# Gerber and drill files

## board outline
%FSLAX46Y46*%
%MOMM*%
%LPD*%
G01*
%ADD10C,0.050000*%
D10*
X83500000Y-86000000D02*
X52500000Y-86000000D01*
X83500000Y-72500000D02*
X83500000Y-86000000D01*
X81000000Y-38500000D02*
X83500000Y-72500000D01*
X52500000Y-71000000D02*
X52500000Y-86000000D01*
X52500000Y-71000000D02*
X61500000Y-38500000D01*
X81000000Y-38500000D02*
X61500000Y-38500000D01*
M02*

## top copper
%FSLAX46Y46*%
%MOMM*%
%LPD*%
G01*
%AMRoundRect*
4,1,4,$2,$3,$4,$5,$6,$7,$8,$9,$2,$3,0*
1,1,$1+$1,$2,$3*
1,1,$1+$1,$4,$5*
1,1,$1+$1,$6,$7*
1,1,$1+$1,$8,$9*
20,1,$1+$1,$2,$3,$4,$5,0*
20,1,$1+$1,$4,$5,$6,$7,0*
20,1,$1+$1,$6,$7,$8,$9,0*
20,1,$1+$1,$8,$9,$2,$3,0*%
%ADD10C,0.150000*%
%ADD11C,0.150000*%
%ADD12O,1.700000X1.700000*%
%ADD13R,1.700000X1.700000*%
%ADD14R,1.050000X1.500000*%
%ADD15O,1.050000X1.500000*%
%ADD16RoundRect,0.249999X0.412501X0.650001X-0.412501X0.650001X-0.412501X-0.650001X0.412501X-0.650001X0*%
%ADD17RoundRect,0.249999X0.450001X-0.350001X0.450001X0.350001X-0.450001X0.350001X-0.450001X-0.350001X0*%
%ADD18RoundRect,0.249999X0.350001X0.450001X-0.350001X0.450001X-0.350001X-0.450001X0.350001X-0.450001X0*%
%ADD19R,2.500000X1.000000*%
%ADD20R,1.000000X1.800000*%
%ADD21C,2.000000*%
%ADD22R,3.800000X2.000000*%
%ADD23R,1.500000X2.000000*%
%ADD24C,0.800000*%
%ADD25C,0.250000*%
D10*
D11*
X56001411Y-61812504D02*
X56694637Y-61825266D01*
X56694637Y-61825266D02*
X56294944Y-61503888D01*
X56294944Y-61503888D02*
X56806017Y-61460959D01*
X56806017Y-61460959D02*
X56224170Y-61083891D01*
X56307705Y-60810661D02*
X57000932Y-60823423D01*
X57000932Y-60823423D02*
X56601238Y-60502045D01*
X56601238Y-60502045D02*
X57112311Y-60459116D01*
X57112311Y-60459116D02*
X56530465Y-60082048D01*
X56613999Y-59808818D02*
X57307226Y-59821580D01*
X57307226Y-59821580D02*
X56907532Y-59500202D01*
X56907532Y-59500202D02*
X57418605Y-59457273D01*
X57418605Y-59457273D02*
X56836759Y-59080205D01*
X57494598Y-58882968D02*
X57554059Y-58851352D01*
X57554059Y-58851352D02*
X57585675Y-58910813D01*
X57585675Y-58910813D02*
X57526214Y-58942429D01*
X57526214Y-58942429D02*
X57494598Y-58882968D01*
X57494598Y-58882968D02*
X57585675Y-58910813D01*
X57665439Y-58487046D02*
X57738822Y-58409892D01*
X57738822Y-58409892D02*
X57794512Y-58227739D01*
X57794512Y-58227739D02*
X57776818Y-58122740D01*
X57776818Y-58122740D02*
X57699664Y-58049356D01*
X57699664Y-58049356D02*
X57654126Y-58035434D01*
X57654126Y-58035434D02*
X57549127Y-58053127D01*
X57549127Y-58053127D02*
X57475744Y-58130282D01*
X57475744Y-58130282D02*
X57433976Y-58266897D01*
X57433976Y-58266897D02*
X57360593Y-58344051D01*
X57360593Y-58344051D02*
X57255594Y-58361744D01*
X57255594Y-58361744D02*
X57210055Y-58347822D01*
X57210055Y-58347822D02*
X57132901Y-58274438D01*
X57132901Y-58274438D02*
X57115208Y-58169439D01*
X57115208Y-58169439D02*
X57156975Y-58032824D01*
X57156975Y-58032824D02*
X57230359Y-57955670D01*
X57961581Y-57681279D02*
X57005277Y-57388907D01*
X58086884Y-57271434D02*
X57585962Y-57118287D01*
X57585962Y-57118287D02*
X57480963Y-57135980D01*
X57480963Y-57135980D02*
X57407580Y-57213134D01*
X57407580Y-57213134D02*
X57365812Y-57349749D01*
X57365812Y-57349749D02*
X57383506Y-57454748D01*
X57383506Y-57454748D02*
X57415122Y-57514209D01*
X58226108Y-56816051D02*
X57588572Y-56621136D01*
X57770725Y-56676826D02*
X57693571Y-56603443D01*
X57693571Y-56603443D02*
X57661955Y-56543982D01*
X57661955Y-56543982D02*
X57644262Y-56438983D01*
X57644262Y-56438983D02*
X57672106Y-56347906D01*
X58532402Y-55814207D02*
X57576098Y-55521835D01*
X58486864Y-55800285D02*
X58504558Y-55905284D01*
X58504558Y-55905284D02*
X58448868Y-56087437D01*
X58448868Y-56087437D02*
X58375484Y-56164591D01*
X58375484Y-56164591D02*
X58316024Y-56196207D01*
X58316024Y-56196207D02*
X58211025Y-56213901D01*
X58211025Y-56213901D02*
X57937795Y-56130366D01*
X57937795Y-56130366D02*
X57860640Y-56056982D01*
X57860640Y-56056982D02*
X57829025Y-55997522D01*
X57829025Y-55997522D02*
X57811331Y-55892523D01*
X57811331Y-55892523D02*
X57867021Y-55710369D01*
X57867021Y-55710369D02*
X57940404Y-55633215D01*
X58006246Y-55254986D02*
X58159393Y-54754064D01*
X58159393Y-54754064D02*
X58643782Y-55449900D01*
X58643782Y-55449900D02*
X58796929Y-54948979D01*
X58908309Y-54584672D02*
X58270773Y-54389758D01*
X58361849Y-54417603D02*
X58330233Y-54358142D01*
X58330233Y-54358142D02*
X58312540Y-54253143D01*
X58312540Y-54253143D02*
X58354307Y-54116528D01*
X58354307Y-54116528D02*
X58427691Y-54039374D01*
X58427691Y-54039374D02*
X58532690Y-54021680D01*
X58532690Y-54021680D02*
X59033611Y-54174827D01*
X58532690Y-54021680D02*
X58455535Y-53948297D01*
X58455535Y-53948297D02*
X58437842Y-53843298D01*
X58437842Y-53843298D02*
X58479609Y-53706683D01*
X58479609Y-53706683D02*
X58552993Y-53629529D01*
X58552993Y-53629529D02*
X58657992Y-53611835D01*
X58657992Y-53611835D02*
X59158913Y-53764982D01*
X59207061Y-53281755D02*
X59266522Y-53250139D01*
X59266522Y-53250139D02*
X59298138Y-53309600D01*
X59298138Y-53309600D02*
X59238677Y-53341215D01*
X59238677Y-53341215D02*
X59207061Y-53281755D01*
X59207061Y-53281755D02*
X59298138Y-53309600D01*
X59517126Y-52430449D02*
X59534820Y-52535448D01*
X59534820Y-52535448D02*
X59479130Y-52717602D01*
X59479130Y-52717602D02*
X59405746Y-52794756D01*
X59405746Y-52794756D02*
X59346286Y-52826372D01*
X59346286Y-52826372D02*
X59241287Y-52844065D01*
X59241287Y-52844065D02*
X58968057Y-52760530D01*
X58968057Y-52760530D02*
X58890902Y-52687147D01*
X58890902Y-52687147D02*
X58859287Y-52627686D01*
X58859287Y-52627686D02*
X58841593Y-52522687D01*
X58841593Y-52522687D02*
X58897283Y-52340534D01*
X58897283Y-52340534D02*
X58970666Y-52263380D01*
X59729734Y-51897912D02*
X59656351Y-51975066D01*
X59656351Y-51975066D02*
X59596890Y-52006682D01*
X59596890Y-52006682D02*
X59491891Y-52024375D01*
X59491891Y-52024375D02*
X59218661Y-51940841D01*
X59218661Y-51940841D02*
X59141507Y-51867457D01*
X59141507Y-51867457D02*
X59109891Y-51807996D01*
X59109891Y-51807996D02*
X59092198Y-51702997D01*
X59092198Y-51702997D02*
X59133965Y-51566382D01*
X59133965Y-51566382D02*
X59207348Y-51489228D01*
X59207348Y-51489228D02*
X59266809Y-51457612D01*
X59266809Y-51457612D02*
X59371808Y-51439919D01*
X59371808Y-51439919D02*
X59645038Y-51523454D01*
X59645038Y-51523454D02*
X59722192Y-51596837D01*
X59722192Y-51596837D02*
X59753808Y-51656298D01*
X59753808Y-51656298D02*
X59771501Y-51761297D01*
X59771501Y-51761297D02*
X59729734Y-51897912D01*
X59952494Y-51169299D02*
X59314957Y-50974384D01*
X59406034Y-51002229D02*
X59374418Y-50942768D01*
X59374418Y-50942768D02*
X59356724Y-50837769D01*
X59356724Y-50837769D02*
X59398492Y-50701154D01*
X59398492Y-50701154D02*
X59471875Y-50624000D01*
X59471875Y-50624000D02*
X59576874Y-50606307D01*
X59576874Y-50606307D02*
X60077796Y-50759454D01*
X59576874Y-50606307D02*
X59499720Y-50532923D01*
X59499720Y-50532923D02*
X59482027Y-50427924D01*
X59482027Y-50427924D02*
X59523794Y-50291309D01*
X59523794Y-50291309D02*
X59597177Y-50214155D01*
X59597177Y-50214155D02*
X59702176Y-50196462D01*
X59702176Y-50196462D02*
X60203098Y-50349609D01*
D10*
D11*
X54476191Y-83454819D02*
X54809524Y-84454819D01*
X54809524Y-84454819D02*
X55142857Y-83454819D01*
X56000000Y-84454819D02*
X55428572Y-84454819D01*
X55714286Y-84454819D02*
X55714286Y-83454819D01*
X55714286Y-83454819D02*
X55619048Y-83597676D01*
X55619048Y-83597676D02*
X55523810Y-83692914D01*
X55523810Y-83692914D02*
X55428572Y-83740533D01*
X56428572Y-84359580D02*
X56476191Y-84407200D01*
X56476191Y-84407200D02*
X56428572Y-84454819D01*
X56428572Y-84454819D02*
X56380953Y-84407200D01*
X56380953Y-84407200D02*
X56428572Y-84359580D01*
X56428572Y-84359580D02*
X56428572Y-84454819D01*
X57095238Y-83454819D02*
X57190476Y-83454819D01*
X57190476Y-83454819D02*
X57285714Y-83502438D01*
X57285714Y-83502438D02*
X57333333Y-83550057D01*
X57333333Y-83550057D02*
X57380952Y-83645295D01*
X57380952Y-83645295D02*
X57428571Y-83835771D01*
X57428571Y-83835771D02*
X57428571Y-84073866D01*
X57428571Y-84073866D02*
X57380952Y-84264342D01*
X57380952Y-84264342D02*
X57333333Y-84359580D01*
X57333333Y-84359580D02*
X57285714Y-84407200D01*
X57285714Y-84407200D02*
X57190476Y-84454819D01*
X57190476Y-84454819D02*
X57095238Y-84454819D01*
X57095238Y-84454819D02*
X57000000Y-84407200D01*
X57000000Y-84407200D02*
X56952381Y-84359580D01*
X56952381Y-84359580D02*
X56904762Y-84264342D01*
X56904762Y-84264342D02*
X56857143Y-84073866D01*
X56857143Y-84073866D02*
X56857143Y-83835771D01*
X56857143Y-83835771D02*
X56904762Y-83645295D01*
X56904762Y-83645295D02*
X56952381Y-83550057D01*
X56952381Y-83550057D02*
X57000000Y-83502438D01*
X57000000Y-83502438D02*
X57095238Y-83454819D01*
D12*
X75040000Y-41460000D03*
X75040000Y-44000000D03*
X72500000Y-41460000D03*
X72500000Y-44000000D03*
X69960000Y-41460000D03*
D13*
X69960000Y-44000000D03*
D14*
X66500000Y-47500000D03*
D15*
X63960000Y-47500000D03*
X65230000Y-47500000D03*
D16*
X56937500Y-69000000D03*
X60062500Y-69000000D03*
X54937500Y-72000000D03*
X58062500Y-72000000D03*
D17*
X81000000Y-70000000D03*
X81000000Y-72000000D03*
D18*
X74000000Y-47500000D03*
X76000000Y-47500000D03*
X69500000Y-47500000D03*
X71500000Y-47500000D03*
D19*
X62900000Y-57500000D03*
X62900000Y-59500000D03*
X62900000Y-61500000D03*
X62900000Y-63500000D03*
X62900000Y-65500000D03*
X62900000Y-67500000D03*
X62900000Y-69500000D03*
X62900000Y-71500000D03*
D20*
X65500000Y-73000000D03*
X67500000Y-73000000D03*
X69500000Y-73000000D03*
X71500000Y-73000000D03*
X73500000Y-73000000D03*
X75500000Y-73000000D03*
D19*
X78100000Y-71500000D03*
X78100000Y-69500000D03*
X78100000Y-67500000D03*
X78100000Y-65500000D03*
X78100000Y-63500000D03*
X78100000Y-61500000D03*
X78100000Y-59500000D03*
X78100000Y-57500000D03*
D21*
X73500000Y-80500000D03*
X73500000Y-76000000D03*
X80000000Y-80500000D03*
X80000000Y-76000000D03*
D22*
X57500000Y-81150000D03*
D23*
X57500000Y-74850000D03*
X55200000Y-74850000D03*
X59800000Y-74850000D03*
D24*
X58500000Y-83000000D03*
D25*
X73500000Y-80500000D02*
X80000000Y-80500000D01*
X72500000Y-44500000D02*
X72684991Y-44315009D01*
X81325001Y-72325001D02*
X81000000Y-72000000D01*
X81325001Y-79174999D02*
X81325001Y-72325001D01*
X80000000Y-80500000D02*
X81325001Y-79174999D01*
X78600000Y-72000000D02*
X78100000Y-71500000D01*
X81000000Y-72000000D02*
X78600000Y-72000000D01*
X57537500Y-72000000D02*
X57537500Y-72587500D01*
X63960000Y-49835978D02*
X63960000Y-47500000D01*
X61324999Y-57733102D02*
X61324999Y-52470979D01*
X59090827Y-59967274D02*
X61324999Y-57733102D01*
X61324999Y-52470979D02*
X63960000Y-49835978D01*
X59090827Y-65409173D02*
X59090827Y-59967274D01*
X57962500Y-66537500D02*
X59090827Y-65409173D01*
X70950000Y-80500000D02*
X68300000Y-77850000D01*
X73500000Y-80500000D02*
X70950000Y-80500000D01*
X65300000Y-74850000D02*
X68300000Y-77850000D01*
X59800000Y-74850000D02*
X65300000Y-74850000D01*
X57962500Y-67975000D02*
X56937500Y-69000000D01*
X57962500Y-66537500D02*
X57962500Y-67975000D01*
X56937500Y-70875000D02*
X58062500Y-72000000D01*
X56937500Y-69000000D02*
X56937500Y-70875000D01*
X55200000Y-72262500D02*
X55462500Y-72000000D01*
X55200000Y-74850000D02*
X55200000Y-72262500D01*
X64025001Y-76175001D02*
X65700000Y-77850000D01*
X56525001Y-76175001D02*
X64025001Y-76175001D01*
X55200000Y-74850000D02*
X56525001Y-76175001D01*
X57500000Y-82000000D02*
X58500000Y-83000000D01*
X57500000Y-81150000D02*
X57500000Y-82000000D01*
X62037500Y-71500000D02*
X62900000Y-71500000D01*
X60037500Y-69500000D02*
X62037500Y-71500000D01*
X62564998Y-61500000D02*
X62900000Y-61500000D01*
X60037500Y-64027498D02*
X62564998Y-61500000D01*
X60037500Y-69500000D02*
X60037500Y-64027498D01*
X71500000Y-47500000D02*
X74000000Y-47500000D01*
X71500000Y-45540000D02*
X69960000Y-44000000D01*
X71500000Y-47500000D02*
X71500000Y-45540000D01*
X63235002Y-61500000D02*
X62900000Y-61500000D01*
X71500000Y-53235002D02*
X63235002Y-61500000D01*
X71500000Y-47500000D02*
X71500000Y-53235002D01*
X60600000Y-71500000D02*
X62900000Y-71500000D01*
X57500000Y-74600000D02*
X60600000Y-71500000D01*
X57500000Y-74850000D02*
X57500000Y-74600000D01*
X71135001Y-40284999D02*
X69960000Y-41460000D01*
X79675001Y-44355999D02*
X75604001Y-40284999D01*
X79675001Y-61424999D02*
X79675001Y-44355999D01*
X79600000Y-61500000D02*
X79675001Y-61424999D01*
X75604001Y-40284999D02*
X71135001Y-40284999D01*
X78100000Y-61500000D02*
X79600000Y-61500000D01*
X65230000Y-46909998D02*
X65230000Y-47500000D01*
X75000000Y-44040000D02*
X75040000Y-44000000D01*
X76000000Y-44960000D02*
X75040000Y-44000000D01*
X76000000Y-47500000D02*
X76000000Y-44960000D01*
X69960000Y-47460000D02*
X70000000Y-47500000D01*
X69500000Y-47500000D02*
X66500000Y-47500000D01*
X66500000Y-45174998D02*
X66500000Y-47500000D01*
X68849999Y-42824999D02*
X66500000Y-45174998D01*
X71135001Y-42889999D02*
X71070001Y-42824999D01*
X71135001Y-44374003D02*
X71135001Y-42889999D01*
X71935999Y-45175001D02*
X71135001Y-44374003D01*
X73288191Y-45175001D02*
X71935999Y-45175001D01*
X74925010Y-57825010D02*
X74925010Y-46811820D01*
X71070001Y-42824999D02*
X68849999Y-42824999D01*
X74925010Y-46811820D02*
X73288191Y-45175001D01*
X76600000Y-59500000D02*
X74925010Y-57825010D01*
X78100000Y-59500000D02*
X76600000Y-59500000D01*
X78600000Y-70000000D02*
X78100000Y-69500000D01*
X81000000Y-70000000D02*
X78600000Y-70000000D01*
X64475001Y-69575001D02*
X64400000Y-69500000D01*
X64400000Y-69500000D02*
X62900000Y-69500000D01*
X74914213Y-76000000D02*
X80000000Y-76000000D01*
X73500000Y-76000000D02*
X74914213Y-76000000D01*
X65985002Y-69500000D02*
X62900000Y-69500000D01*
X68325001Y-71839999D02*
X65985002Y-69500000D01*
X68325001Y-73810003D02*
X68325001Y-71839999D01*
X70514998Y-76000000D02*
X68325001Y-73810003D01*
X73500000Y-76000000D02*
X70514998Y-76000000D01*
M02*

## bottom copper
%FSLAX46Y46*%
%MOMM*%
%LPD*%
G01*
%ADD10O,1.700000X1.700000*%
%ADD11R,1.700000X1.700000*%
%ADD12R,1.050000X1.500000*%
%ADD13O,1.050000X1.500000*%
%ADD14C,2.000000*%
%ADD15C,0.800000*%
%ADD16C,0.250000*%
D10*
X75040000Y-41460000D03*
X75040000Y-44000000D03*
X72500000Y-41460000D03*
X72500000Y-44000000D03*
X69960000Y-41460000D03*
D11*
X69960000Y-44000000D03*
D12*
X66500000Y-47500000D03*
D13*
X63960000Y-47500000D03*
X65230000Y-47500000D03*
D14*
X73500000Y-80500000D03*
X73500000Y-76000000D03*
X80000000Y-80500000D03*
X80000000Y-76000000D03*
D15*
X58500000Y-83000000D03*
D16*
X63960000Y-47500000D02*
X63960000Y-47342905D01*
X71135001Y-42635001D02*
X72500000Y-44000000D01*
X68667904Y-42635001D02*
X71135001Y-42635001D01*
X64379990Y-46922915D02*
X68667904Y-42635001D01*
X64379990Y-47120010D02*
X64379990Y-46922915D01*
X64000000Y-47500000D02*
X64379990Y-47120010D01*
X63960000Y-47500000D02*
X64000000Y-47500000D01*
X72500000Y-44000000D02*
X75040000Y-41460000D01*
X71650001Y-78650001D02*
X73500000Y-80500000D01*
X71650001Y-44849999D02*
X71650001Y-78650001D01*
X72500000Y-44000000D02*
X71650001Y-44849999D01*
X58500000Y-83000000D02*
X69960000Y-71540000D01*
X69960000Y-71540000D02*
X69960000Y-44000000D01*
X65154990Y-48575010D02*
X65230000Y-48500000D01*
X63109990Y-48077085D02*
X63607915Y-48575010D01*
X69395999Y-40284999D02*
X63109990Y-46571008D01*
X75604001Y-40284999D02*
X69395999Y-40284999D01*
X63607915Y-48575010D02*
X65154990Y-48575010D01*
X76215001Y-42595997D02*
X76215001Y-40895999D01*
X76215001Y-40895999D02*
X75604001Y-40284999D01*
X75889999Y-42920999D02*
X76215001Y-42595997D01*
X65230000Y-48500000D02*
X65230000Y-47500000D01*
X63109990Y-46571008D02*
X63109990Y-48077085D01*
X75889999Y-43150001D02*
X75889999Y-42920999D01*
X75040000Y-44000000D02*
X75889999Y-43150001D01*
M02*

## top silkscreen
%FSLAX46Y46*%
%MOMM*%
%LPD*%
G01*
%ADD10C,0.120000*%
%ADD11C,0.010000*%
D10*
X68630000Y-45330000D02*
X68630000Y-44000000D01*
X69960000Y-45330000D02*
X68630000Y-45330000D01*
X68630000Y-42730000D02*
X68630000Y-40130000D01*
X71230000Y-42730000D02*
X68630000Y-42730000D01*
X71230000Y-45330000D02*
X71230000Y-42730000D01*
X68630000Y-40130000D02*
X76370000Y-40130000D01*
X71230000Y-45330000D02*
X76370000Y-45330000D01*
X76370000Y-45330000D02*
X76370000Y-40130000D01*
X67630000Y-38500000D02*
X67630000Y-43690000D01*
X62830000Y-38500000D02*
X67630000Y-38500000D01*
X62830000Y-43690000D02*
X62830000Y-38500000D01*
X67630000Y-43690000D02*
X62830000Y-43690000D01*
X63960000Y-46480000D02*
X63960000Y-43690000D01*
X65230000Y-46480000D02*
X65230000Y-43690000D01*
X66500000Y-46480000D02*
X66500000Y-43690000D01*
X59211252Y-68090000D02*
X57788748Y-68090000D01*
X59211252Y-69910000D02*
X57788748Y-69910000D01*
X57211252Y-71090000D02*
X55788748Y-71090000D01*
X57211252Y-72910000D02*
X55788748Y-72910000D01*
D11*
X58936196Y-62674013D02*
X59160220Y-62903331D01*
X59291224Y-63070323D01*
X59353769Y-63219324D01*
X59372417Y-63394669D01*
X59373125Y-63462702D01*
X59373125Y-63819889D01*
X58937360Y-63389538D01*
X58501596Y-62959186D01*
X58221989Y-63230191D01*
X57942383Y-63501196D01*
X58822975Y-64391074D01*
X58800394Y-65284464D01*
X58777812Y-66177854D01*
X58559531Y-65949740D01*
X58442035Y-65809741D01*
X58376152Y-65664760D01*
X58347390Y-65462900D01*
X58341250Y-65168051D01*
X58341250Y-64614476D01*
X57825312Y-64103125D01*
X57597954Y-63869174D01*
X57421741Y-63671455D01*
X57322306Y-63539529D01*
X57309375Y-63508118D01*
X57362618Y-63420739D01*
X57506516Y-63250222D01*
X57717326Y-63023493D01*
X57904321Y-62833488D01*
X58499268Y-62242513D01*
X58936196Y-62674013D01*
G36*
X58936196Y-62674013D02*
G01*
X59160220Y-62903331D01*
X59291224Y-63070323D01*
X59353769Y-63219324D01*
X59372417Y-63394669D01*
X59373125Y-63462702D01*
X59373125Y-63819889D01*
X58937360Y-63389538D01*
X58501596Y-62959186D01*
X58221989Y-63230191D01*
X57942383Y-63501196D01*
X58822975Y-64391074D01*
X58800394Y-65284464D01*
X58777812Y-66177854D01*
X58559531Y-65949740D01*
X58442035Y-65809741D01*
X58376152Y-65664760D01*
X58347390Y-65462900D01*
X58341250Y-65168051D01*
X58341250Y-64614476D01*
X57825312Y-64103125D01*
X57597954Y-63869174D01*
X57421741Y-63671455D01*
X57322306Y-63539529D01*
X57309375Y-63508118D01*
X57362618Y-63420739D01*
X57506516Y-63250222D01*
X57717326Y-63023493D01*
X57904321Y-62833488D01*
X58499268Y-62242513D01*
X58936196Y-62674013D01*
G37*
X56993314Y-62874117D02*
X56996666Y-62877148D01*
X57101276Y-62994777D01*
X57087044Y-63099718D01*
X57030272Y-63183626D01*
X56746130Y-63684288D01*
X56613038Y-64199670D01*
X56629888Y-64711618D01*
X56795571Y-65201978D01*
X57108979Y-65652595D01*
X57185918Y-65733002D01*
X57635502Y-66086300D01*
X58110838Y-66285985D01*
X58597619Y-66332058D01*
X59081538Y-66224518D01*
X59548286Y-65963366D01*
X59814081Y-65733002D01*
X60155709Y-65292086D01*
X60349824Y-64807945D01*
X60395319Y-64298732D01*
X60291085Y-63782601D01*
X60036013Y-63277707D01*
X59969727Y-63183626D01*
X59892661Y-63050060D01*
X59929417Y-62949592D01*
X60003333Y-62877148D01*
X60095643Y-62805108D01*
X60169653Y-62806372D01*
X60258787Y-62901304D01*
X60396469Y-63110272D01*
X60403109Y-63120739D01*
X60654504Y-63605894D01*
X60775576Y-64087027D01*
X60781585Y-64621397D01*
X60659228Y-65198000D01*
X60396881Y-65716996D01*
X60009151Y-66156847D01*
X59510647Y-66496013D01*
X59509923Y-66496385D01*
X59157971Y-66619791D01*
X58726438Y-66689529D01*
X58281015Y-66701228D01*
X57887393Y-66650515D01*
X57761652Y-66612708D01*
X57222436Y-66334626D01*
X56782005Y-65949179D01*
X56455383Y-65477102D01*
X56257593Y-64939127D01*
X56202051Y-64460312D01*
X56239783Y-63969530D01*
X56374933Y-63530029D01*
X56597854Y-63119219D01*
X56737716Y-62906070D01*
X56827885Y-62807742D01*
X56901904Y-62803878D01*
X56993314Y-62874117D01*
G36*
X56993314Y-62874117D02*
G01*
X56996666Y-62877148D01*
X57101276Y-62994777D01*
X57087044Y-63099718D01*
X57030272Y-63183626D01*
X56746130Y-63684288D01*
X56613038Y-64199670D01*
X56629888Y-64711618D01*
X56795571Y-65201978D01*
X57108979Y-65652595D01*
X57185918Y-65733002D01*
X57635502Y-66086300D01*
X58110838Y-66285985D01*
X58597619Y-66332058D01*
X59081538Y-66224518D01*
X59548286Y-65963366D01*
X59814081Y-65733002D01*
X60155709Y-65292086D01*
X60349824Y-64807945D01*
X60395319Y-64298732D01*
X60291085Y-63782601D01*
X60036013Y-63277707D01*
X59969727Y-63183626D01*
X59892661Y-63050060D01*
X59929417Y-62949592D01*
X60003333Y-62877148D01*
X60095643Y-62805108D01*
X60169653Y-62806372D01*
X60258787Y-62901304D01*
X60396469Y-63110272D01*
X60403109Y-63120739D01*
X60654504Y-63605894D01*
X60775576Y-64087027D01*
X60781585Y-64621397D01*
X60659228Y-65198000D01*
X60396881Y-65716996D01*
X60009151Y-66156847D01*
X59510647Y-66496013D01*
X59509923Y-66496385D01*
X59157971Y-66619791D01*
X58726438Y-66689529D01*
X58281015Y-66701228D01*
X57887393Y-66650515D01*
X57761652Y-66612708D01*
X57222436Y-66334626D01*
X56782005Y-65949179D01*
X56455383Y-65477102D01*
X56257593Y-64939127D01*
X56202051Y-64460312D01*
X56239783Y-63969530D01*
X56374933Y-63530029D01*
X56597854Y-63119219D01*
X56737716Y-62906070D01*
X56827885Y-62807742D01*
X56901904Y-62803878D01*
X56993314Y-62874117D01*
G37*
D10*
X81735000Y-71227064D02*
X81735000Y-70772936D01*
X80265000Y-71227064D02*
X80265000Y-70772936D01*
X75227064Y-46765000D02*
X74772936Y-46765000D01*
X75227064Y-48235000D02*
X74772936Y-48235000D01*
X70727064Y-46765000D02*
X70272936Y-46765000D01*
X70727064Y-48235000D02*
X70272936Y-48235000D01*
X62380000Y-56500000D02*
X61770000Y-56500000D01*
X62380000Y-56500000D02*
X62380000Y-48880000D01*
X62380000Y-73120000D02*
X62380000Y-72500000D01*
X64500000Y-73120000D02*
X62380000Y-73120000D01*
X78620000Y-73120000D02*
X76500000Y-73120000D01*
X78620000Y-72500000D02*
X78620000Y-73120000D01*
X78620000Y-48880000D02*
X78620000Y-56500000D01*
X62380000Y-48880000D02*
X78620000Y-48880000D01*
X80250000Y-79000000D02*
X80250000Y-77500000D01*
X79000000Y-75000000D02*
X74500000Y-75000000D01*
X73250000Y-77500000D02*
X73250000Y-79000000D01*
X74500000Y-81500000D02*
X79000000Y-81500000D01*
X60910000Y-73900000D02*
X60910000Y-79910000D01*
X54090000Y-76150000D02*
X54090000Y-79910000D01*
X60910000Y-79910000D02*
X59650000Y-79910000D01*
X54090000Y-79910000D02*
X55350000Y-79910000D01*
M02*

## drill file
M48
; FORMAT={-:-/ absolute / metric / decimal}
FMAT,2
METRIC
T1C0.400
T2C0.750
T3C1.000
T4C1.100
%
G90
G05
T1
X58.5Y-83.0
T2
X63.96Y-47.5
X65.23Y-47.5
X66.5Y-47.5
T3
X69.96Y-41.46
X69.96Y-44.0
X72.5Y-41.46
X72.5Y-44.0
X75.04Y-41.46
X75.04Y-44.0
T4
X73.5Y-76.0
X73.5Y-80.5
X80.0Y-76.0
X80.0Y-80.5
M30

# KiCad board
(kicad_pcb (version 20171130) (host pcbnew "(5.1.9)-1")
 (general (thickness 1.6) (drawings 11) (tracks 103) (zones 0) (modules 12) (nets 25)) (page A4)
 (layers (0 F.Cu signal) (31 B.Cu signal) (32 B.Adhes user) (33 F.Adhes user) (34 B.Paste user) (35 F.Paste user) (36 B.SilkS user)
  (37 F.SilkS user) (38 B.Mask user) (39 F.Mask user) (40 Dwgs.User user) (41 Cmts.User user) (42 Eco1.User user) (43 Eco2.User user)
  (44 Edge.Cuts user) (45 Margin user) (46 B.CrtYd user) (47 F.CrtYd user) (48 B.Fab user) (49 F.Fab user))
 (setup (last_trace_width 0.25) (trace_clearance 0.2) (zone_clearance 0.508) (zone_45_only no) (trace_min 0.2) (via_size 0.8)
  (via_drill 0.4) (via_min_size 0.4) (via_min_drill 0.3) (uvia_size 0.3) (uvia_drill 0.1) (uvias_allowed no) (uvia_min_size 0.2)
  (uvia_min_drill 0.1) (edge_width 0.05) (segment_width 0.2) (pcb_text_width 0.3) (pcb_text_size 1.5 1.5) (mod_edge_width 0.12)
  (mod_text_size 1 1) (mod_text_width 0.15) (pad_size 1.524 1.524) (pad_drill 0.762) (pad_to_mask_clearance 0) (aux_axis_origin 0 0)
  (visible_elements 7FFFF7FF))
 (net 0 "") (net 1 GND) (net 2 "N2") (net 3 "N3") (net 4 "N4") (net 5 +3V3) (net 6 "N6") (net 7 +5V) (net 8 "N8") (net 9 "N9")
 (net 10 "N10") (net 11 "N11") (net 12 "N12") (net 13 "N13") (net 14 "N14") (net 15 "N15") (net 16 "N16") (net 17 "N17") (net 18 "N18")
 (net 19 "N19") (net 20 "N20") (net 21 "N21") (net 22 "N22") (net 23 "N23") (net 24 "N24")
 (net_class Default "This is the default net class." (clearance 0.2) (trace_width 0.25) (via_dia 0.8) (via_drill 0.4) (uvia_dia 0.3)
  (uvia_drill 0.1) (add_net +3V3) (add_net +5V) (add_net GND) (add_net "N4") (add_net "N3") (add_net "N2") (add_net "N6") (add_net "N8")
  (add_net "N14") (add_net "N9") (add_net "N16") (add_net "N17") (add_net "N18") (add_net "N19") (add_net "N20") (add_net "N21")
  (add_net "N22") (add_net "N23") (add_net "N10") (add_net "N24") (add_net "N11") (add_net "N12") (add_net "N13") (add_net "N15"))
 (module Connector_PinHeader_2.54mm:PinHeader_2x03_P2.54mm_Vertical (layer F.Cu) (at 69.96 44 90)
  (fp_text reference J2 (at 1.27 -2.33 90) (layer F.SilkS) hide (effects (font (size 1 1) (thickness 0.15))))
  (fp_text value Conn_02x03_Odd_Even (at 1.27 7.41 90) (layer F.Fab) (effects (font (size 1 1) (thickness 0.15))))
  (fp_line (start -1.33 -1.33) (end 0 -1.33) (layer F.SilkS) (width 0.12))
  (fp_line (start -1.33 0) (end -1.33 -1.33) (layer F.SilkS) (width 0.12))
  (fp_line (start 1.27 -1.33) (end 3.87 -1.33) (layer F.SilkS) (width 0.12))
  (fp_line (start 1.27 1.27) (end 1.27 -1.33) (layer F.SilkS) (width 0.12))
  (fp_line (start -1.33 1.27) (end 1.27 1.27) (layer F.SilkS) (width 0.12))
  (fp_line (start 3.87 -1.33) (end 3.87 6.41) (layer F.SilkS) (width 0.12))
  (fp_line (start -1.33 1.27) (end -1.33 6.41) (layer F.SilkS) (width 0.12))
  (fp_line (start -1.33 6.41) (end 3.87 6.41) (layer F.SilkS) (width 0.12))
  (pad 6 thru_hole oval (at 2.54 5.08 90) (size 1.7 1.7) (drill 1) (layers *.Cu *.Mask) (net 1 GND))
  (pad 5 thru_hole oval (at 0 5.08 90) (size 1.7 1.7) (drill 1) (layers *.Cu *.Mask) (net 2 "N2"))
  (pad 4 thru_hole oval (at 2.54 2.54 90) (size 1.7 1.7) (drill 1) (layers *.Cu *.Mask) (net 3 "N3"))
  (pad 3 thru_hole oval (at 0 2.54 90) (size 1.7 1.7) (drill 1) (layers *.Cu *.Mask) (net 1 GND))
  (pad 2 thru_hole oval (at 2.54 0 90) (size 1.7 1.7) (drill 1) (layers *.Cu *.Mask) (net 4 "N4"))
  (pad 1 thru_hole rect (at 0 0 90) (size 1.7 1.7) (drill 1) (layers *.Cu *.Mask) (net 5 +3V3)))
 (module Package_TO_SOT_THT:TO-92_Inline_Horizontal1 (layer F.Cu) (at 66.5 47.5 180)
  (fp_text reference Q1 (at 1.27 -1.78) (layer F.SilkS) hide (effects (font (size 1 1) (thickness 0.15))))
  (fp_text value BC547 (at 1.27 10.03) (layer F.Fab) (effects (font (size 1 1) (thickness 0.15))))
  (fp_line (start -1.13 9) (end -1.13 3.81) (layer F.SilkS) (width 0.12))
  (fp_line (start 3.67 9) (end -1.13 9) (layer F.SilkS) (width 0.12))
  (fp_line (start 3.67 3.81) (end 3.67 9) (layer F.SilkS) (width 0.12))
  (fp_line (start -1.13 3.81) (end 3.67 3.81) (layer F.SilkS) (width 0.12))
  (fp_line (start 2.54 1.02) (end 2.54 3.81) (layer F.SilkS) (width 0.12))
  (fp_line (start 1.27 1.02) (end 1.27 3.81) (layer F.SilkS) (width 0.12))
  (fp_line (start 0 1.02) (end 0 3.81) (layer F.SilkS) (width 0.12))
  (pad 1 thru_hole rect (at 0 0 180) (size 1.05 1.5) (drill 0.75) (layers *.Cu *.Mask) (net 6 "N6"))
  (pad 3 thru_hole oval (at 2.54 0 180) (size 1.05 1.5) (drill 0.75) (layers *.Cu *.Mask) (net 1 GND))
  (pad 2 thru_hole oval (at 1.27 0 180) (size 1.05 1.5) (drill 0.75) (layers *.Cu *.Mask) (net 2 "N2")))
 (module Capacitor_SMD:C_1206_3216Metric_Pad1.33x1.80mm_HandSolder (layer F.Cu) (at 58.5 69 180)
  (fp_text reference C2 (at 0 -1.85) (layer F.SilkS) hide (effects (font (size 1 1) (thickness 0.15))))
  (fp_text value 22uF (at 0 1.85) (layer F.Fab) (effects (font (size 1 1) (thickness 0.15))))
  (fp_line (start -0.711252 0.91) (end 0.711252 0.91) (layer F.SilkS) (width 0.12))
  (fp_line (start -0.711252 -0.91) (end 0.711252 -0.91) (layer F.SilkS) (width 0.12))
  (pad 2 smd roundrect (at 1.5625 0 180) (size 1.325 1.8) (layers F.Cu F.Paste F.Mask) (roundrect_rratio 0.1886784905660377) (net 1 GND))
  (pad 1 smd roundrect (at -1.5625 0 180) (size 1.325 1.8) (layers F.Cu F.Paste F.Mask) (roundrect_rratio 0.1886784905660377) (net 5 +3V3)))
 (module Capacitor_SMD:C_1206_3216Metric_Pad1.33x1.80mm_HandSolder (layer F.Cu) (at 56.5 72 180)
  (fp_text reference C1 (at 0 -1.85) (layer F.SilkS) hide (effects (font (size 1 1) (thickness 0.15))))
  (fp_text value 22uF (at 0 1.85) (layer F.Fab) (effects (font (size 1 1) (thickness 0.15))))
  (fp_line (start -0.711252 0.91) (end 0.711252 0.91) (layer F.SilkS) (width 0.12))
  (fp_line (start -0.711252 -0.91) (end 0.711252 -0.91) (layer F.SilkS) (width 0.12))
  (pad 2 smd roundrect (at 1.5625 0 180) (size 1.325 1.8) (layers F.Cu F.Paste F.Mask) (roundrect_rratio 0.1886784905660377) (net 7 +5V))
  (pad 1 smd roundrect (at -1.5625 0 180) (size 1.325 1.8) (layers F.Cu F.Paste F.Mask) (roundrect_rratio 0.1886784905660377) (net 1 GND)))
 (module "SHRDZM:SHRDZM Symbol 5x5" (layer F.Cu) (at 58.5 64.5)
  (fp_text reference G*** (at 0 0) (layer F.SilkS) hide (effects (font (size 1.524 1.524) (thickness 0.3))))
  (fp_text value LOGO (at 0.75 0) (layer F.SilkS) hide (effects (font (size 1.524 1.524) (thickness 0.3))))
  (fp_poly
   (pts (xy 0.436196 -1.825987) (xy 0.66022 -1.596669) (xy 0.791224 -1.429677) (xy 0.853769 -1.280676) (xy 0.872417 -1.105331)
    (xy 0.873125 -1.037298) (xy 0.873125 -0.680111) (xy 0.43736 -1.110462) (xy 0.001596 -1.540814) (xy -0.278011 -1.269809)
    (xy -0.557617 -0.998804) (xy 0.322975 -0.108926) (xy 0.300394 0.784464) (xy 0.277812 1.677854) (xy 0.059531 1.44974)
    (xy -0.057965 1.309741) (xy -0.123848 1.16476) (xy -0.15261 0.9629) (xy -0.15875 0.668051) (xy -0.15875 0.114476)
    (xy -0.674688 -0.396875) (xy -0.902046 -0.630826) (xy -1.078259 -0.828545) (xy -1.177694 -0.960471) (xy -1.190625 -0.991882)
    (xy -1.137382 -1.079261) (xy -0.993484 -1.249778) (xy -0.782674 -1.476507) (xy -0.595679 -1.666512) (xy -0.000732 -2.257487)
    (xy 0.436196 -1.825987))
   (layer F.SilkS) (width 0.01))
  (fp_poly
   (pts (xy -1.506686 -1.625883) (xy -1.503334 -1.622852) (xy -1.398724 -1.505223) (xy -1.412956 -1.400282) (xy -1.469728 -1.316374)
    (xy -1.75387 -0.815712) (xy -1.886962 -0.30033) (xy -1.870112 0.211618) (xy -1.704429 0.701978) (xy -1.391021 1.152595)
    (xy -1.314082 1.233002) (xy -0.864498 1.5863) (xy -0.389162 1.785985) (xy 0.097619 1.832058) (xy 0.581538 1.724518)
    (xy 1.048286 1.463366) (xy 1.314081 1.233002) (xy 1.655709 0.792086) (xy 1.849824 0.307945) (xy 1.895319 -0.201268)
    (xy 1.791085 -0.717399) (xy 1.536013 -1.222293) (xy 1.469727 -1.316374) (xy 1.392661 -1.44994) (xy 1.429417 -1.550408)
    (xy 1.503333 -1.622852) (xy 1.595643 -1.694892) (xy 1.669653 -1.693628) (xy 1.758787 -1.598696) (xy 1.896469 -1.389728)
    (xy 1.903109 -1.379261) (xy 2.154504 -0.894106) (xy 2.275576 -0.412973) (xy 2.281585 0.121397) (xy 2.159228 0.698)
    (xy 1.896881 1.216996) (xy 1.509151 1.656847) (xy 1.010647 1.996013) (xy 1.009923 1.996385) (xy 0.657971 2.119791)
    (xy 0.226438 2.189529) (xy -0.218985 2.201228) (xy -0.612607 2.150515) (xy -0.738348 2.112708) (xy -1.277564 1.834626)
    (xy -1.717995 1.449179) (xy -2.044617 0.977102) (xy -2.242407 0.439127) (xy -2.297949 -0.039688) (xy -2.260217 -0.53047)
    (xy -2.125067 -0.969971) (xy -1.902146 -1.380781) (xy -1.762284 -1.59393) (xy -1.672115 -1.692258) (xy -1.598096 -1.696122)
    (xy -1.506686 -1.625883))
   (layer F.SilkS) (width 0.01)))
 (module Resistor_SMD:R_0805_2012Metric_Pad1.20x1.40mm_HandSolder (layer F.Cu) (at 81 71 90)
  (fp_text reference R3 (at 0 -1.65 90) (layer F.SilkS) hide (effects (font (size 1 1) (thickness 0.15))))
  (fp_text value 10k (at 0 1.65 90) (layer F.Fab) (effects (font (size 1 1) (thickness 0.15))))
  (fp_line (start -0.227064 0.735) (end 0.227064 0.735) (layer F.SilkS) (width 0.12))
  (fp_line (start -0.227064 -0.735) (end 0.227064 -0.735) (layer F.SilkS) (width 0.12))
  (pad 2 smd roundrect (at 1 0 90) (size 1.2 1.4) (layers F.Cu F.Paste F.Mask) (roundrect_rratio 0.2083325) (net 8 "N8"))
  (pad 1 smd roundrect (at -1 0 90) (size 1.2 1.4) (layers F.Cu F.Paste F.Mask) (roundrect_rratio 0.2083325) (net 1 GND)))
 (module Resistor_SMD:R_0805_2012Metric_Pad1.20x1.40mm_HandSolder (layer F.Cu) (at 75 47.5 180)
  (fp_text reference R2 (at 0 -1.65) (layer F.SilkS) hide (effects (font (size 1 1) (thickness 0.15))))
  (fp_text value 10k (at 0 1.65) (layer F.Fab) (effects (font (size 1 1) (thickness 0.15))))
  (fp_line (start -0.227064 0.735) (end 0.227064 0.735) (layer F.SilkS) (width 0.12))
  (fp_line (start -0.227064 -0.735) (end 0.227064 -0.735) (layer F.SilkS) (width 0.12))
  (pad 2 smd roundrect (at 1 0 180) (size 1.2 1.4) (layers F.Cu F.Paste F.Mask) (roundrect_rratio 0.2083325) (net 5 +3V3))
  (pad 1 smd roundrect (at -1 0 180) (size 1.2 1.4) (layers F.Cu F.Paste F.Mask) (roundrect_rratio 0.2083325) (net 2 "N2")))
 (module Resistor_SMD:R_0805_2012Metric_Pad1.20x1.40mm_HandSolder (layer F.Cu) (at 70.5 47.5 180)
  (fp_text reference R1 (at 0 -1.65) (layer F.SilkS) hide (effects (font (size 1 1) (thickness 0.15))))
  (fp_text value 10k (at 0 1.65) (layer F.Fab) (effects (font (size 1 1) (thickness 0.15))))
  (fp_line (start -0.227064 0.735) (end 0.227064 0.735) (layer F.SilkS) (width 0.12))
  (fp_line (start -0.227064 -0.735) (end 0.227064 -0.735) (layer F.SilkS) (width 0.12))
  (pad 2 smd roundrect (at 1 0 180) (size 1.2 1.4) (layers F.Cu F.Paste F.Mask) (roundrect_rratio 0.2083325) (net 6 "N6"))
  (pad 1 smd roundrect (at -1 0 180) (size 1.2 1.4) (layers F.Cu F.Paste F.Mask) (roundrect_rratio 0.2083325) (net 5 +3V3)))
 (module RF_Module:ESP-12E (layer F.Cu) (at 70.5 61)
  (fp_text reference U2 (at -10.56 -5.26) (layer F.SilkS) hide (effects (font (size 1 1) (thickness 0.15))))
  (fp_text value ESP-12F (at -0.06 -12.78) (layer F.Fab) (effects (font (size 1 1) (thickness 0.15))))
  (fp_line (start -8.12 -4.5) (end -8.73 -4.5) (layer F.SilkS) (width 0.12))
  (fp_line (start -8.12 -4.5) (end -8.12 -12.12) (layer F.SilkS) (width 0.12))
  (fp_line (start -8.12 12.12) (end -8.12 11.5) (layer F.SilkS) (width 0.12))
  (fp_line (start -6 12.12) (end -8.12 12.12) (layer F.SilkS) (width 0.12))
  (fp_line (start 8.12 12.12) (end 6 12.12) (layer F.SilkS) (width 0.12))
  (fp_line (start 8.12 11.5) (end 8.12 12.12) (layer F.SilkS) (width 0.12))
  (fp_line (start 8.12 -12.12) (end 8.12 -4.5) (layer F.SilkS) (width 0.12))
  (fp_line (start -8.12 -12.12) (end 8.12 -12.12) (layer F.SilkS) (width 0.12))
  (pad 1 smd rect (at -7.6 -3.5) (size 2.5 1) (layers F.Cu F.Paste F.Mask) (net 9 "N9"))
  (pad 2 smd rect (at -7.6 -1.5) (size 2.5 1) (layers F.Cu F.Paste F.Mask) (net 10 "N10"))
  (pad 3 smd rect (at -7.6 0.5) (size 2.5 1) (layers F.Cu F.Paste F.Mask) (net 5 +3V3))
  (pad 4 smd rect (at -7.6 2.5) (size 2.5 1) (layers F.Cu F.Paste F.Mask) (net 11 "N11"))
  (pad 5 smd rect (at -7.6 4.5) (size 2.5 1) (layers F.Cu F.Paste F.Mask) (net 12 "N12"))
  (pad 6 smd rect (at -7.6 6.5) (size 2.5 1) (layers F.Cu F.Paste F.Mask) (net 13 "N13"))
  (pad 7 smd rect (at -7.6 8.5) (size 2.5 1) (layers F.Cu F.Paste F.Mask) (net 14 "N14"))
  (pad 8 smd rect (at -7.6 10.5) (size 2.5 1) (layers F.Cu F.Paste F.Mask) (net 5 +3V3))
  (pad 9 smd rect (at -5 12) (size 1 1.8) (layers F.Cu F.Paste F.Mask) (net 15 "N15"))
  (pad 10 smd rect (at -3 12) (size 1 1.8) (layers F.Cu F.Paste F.Mask) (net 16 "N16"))
  (pad 11 smd rect (at -1 12) (size 1 1.8) (layers F.Cu F.Paste F.Mask) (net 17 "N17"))
  (pad 12 smd rect (at 1 12) (size 1 1.8) (layers F.Cu F.Paste F.Mask) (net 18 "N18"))
  (pad 13 smd rect (at 3 12) (size 1 1.8) (layers F.Cu F.Paste F.Mask) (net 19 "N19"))
  (pad 14 smd rect (at 5 12) (size 1 1.8) (layers F.Cu F.Paste F.Mask) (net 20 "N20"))
  (pad 15 smd rect (at 7.6 10.5) (size 2.5 1) (layers F.Cu F.Paste F.Mask) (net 1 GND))
  (pad 16 smd rect (at 7.6 8.5) (size 2.5 1) (layers F.Cu F.Paste F.Mask) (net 8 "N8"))
  (pad 17 smd rect (at 7.6 6.5) (size 2.5 1) (layers F.Cu F.Paste F.Mask) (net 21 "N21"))
  (pad 18 smd rect (at 7.6 4.5) (size 2.5 1) (layers F.Cu F.Paste F.Mask) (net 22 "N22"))
  (pad 19 smd rect (at 7.6 2.5) (size 2.5 1) (layers F.Cu F.Paste F.Mask) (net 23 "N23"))
  (pad 20 smd rect (at 7.6 0.5) (size 2.5 1) (layers F.Cu F.Paste F.Mask) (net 4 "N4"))
  (pad 21 smd rect (at 7.6 -1.5) (size 2.5 1) (layers F.Cu F.Paste F.Mask) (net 6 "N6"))
  (pad 22 smd rect (at 7.6 -3.5) (size 2.5 1) (layers F.Cu F.Paste F.Mask) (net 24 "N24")))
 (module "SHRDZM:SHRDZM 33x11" (layer B.Cu) (at 66 65 270)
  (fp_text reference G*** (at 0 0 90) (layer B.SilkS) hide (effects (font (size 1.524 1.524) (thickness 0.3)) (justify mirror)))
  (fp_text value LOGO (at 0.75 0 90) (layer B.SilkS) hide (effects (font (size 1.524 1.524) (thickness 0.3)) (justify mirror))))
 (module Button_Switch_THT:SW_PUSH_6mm (layer F.Cu) (at 73.5 76)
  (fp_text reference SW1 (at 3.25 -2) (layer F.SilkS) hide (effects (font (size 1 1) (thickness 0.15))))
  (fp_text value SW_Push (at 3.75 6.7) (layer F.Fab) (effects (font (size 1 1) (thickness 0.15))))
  (fp_line (start 6.75 3) (end 6.75 1.5) (layer F.SilkS) (width 0.12))
  (fp_line (start 5.5 -1) (end 1 -1) (layer F.SilkS) (width 0.12))
  (fp_line (start -0.25 1.5) (end -0.25 3) (layer F.SilkS) (width 0.12))
  (fp_line (start 1 5.5) (end 5.5 5.5) (layer F.SilkS) (width 0.12))
  (pad 2 thru_hole circle (at 0 4.5 90) (size 2 2) (drill 1.1) (layers *.Cu *.Mask) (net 1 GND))
  (pad 1 thru_hole circle (at 0 0 90) (size 2 2) (drill 1.1) (layers *.Cu *.Mask) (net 14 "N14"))
  (pad 2 thru_hole circle (at 6.5 4.5 90) (size 2 2) (drill 1.1) (layers *.Cu *.Mask) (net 1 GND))
  (pad 1 thru_hole circle (at 6.5 0 90) (size 2 2) (drill 1.1) (layers *.Cu *.Mask) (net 14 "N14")))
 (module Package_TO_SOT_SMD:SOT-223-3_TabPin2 (layer F.Cu) (at 57.5 78 270)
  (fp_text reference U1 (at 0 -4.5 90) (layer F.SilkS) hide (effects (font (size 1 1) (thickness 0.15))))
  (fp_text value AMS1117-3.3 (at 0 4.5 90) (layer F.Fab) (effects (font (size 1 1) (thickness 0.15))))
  (fp_line (start -4.1 -3.41) (end 1.91 -3.41) (layer F.SilkS) (width 0.12))
  (fp_line (start -1.85 3.41) (end 1.91 3.41) (layer F.SilkS) (width 0.12))
  (fp_line (start 1.91 -3.41) (end 1.91 -2.15) (layer F.SilkS) (width 0.12))
  (fp_line (start 1.91 3.41) (end 1.91 2.15) (layer F.SilkS) (width 0.12))
  (pad 2 smd rect (at 3.15 0 270) (size 2 3.8) (layers F.Cu F.Paste F.Mask) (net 5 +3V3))
  (pad 2 smd rect (at -3.15 0 270) (size 2 1.5) (layers F.Cu F.Paste F.Mask) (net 5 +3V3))
  (pad 3 smd rect (at -3.15 2.3 270) (size 2 1.5) (layers F.Cu F.Paste F.Mask) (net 7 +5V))
  (pad 1 smd rect (at -3.15 -2.3 270) (size 2 1.5) (layers F.Cu F.Paste F.Mask) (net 1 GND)))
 (gr_line (start 83.5 86) (end 52.5 86) (layer Edge.Cuts) (width 0.05))
 (gr_line (start 83.5 72.5) (end 83.5 86) (layer Edge.Cuts) (width 0.05))
 (gr_line (start 81 38.5) (end 83.5 72.5) (layer Edge.Cuts) (width 0.05))
 (gr_line (start 52.5 71) (end 52.5 86) (layer Edge.Cuts) (width 0.05))
 (gr_line (start 52.5 71) (end 61.5 38.5) (layer Edge.Cuts) (width 0.05))
 (gr_line (start 81 38.5) (end 61.5 38.5) (layer Edge.Cuts) (width 0.05))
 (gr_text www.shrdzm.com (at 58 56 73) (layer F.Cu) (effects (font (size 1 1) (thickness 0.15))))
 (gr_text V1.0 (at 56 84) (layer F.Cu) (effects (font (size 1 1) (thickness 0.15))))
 (segment (start 73.5 80.5) (end 80 80.5) (width 0.25) (layer F.Cu) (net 1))
 (segment (start 72.5 44.5) (end 72.684991 44.315009) (width 0.25) (layer F.Cu) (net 1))
 (segment (start 63.96 47.5) (end 63.96 47.342905) (width 0.25) (layer B.Cu) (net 1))
 (segment (start 81.325001 72.325001) (end 81 72) (width 0.25) (layer F.Cu) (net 1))
 (segment (start 81.325001 79.174999) (end 81.325001 72.325001) (width 0.25) (layer F.Cu) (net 1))
 (segment (start 80 80.5) (end 81.325001 79.174999) (width 0.25) (layer F.Cu) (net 1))
 (segment (start 78.6 72) (end 78.1 71.5) (width 0.25) (layer F.Cu) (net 1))
 (segment (start 81 72) (end 78.6 72) (width 0.25) (layer F.Cu) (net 1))
 (segment (start 57.5375 72) (end 57.5375 72.5875) (width 0.25) (layer F.Cu) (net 1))
 (segment (start 63.96 49.835978) (end 63.96 47.5) (width 0.25) (layer F.Cu) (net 1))
 (segment (start 61.324999 57.733102) (end 61.324999 52.470979) (width 0.25) (layer F.Cu) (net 1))
 (segment (start 59.090827 59.967274) (end 61.324999 57.733102) (width 0.25) (layer F.Cu) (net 1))
 (segment (start 61.324999 52.470979) (end 63.96 49.835978) (width 0.25) (layer F.Cu) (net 1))
 (segment (start 59.090827 65.409173) (end 59.090827 59.967274) (width 0.25) (layer F.Cu) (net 1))
 (segment (start 57.9625 66.5375) (end 59.090827 65.409173) (width 0.25) (layer F.Cu) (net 1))
 (segment (start 71.135001 42.635001) (end 72.5 44) (width 0.25) (layer B.Cu) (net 1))
 (segment (start 68.667904 42.635001) (end 71.135001 42.635001) (width 0.25) (layer B.Cu) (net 1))
 (segment (start 64.37999 46.922915) (end 68.667904 42.635001) (width 0.25) (layer B.Cu) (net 1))
 (segment (start 64.37999 47.12001) (end 64.37999 46.922915) (width 0.25) (layer B.Cu) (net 1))
 (segment (start 64 47.5) (end 64.37999 47.12001) (width 0.25) (layer B.Cu) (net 1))
 (segment (start 63.96 47.5) (end 64 47.5) (width 0.25) (layer B.Cu) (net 1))
 (segment (start 72.5 44) (end 75.04 41.46) (width 0.25) (layer B.Cu) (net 1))
 (segment (start 71.650001 78.650001) (end 73.5 80.5) (width 0.25) (layer B.Cu) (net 1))
 (segment (start 71.650001 44.849999) (end 71.650001 78.650001) (width 0.25) (layer B.Cu) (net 1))
 (segment (start 72.5 44) (end 71.650001 44.849999) (width 0.25) (layer B.Cu) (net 1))
 (segment (start 70.95 80.5) (end 68.3 77.85) (width 0.25) (layer F.Cu) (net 1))
 (segment (start 73.5 80.5) (end 70.95 80.5) (width 0.25) (layer F.Cu) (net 1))
 (segment (start 65.3 74.85) (end 68.3 77.85) (width 0.25) (layer F.Cu) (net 1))
 (segment (start 59.8 74.85) (end 65.3 74.85) (width 0.25) (layer F.Cu) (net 1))
 (segment (start 57.9625 67.975) (end 56.9375 69) (width 0.25) (layer F.Cu) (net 1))
 (segment (start 57.9625 66.5375) (end 57.9625 67.975) (width 0.25) (layer F.Cu) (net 1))
 (segment (start 56.9375 70.875) (end 58.0625 72) (width 0.25) (layer F.Cu) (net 1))
 (segment (start 56.9375 69) (end 56.9375 70.875) (width 0.25) (layer F.Cu) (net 1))
 (segment (start 55.2 72.2625) (end 55.4625 72) (width 0.25) (layer F.Cu) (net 7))
 (segment (start 55.2 74.85) (end 55.2 72.2625) (width 0.25) (layer F.Cu) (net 7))
 (segment (start 64.025001 76.175001) (end 65.7 77.85) (width 0.25) (layer F.Cu) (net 7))
 (segment (start 56.525001 76.175001) (end 64.025001 76.175001) (width 0.25) (layer F.Cu) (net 7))
 (segment (start 55.2 74.85) (end 56.525001 76.175001) (width 0.25) (layer F.Cu) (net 7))
 (via (at 58.5 83) (size 0.8) (drill 0.4) (layers F.Cu B.Cu) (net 5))
 (segment (start 57.5 82) (end 58.5 83) (width 0.25) (layer F.Cu) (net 5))
 (segment (start 57.5 81.15) (end 57.5 82) (width 0.25) (layer F.Cu) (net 5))
 (segment (start 62.0375 71.5) (end 62.9 71.5) (width 0.25) (layer F.Cu) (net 5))
 (segment (start 60.0375 69.5) (end 62.0375 71.5) (width 0.25) (layer F.Cu) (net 5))
 (segment (start 62.564998 61.5) (end 62.9 61.5) (width 0.25) (layer F.Cu) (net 5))
 (segment (start 60.0375 64.027498) (end 62.564998 61.5) (width 0.25) (layer F.Cu) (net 5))
 (segment (start 60.0375 69.5) (end 60.0375 64.027498) (width 0.25) (layer F.Cu) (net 5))
 (segment (start 71.5 47.5) (end 74 47.5) (width 0.25) (layer F.Cu) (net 5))
 (segment (start 71.5 45.54) (end 69.96 44) (width 0.25) (layer F.Cu) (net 5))
 (segment (start 71.5 47.5) (end 71.5 45.54) (width 0.25) (layer F.Cu) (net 5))
 (segment (start 63.235002 61.5) (end 62.9 61.5) (width 0.25) (layer F.Cu) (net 5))
 (segment (start 71.5 53.235002) (end 63.235002 61.5) (width 0.25) (layer F.Cu) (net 5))
 (segment (start 71.5 47.5) (end 71.5 53.235002) (width 0.25) (layer F.Cu) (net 5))
 (segment (start 58.5 83) (end 69.96 71.54) (width 0.25) (layer B.Cu) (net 5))
 (segment (start 60.6 71.5) (end 62.9 71.5) (width 0.25) (layer F.Cu) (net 5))
 (segment (start 57.5 74.6) (end 60.6 71.5) (width 0.25) (layer F.Cu) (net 5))
 (segment (start 57.5 74.85) (end 57.5 74.6) (width 0.25) (layer F.Cu) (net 5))
 (segment (start 69.96 71.54) (end 69.96 44) (width 0.25) (layer B.Cu) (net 5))
 (segment (start 71.135001 40.284999) (end 69.96 41.46) (width 0.25) (layer F.Cu) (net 4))
 (segment (start 79.675001 44.355999) (end 75.604001 40.284999) (width 0.25) (layer F.Cu) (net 4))
 (segment (start 79.675001 61.424999) (end 79.675001 44.355999) (width 0.25) (layer F.Cu) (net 4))
 (segment (start 79.6 61.5) (end 79.675001 61.424999) (width 0.25) (layer F.Cu) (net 4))
 (segment (start 75.604001 40.284999) (end 71.135001 40.284999) (width 0.25) (layer F.Cu) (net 4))
 (segment (start 78.1 61.5) (end 79.6 61.5) (width 0.25) (layer F.Cu) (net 4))
 (segment (start 65.23 46.909998) (end 65.23 47.5) (width 0.25) (layer F.Cu) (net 2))
 (segment (start 75 44.04) (end 75.04 44) (width 0.25) (layer F.Cu) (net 2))
 (segment (start 65.15499 48.57501) (end 65.23 48.5) (width 0.25) (layer B.Cu) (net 2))
 (segment (start 63.10999 48.077085) (end 63.607915 48.57501) (width 0.25) (layer B.Cu) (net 2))
 (segment (start 69.395999 40.284999) (end 63.10999 46.571008) (width 0.25) (layer B.Cu) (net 2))
 (segment (start 75.604001 40.284999) (end 69.395999 40.284999) (width 0.25) (layer B.Cu) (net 2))
 (segment (start 63.607915 48.57501) (end 65.15499 48.57501) (width 0.25) (layer B.Cu) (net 2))
 (segment (start 76.215001 42.595997) (end 76.215001 40.895999) (width 0.25) (layer B.Cu) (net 2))
 (segment (start 76.215001 40.895999) (end 75.604001 40.284999) (width 0.25) (layer B.Cu) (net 2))
 (segment (start 75.889999 42.920999) (end 76.215001 42.595997) (width 0.25) (layer B.Cu) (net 2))
 (segment (start 65.23 48.5) (end 65.23 47.5) (width 0.25) (layer B.Cu) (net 2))
 (segment (start 63.10999 46.571008) (end 63.10999 48.077085) (width 0.25) (layer B.Cu) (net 2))
 (segment (start 75.889999 43.150001) (end 75.889999 42.920999) (width 0.25) (layer B.Cu) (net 2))
 (segment (start 75.04 44) (end 75.889999 43.150001) (width 0.25) (layer B.Cu) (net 2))
 (segment (start 76 44.96) (end 75.04 44) (width 0.25) (layer F.Cu) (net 2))
 (segment (start 76 47.5) (end 76 44.96) (width 0.25) (layer F.Cu) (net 2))
 (segment (start 69.96 47.46) (end 70 47.5) (width 0.25) (layer F.Cu) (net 6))
 (segment (start 69.5 47.5) (end 66.5 47.5) (width 0.25) (layer F.Cu) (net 6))
 (segment (start 66.5 45.174998) (end 66.5 47.5) (width 0.25) (layer F.Cu) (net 6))
 (segment (start 68.849999 42.824999) (end 66.5 45.174998) (width 0.25) (layer F.Cu) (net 6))
 (segment (start 71.135001 42.889999) (end 71.070001 42.824999) (width 0.25) (layer F.Cu) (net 6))
 (segment (start 71.135001 44.374003) (end 71.135001 42.889999) (width 0.25) (layer F.Cu) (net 6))
 (segment (start 71.935999 45.175001) (end 71.135001 44.374003) (width 0.25) (layer F.Cu) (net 6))
 (segment (start 73.288191 45.175001) (end 71.935999 45.175001) (width 0.25) (layer F.Cu) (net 6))
 (segment (start 74.92501 57.82501) (end 74.92501 46.81182) (width 0.25) (layer F.Cu) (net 6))
 (segment (start 71.070001 42.824999) (end 68.849999 42.824999) (width 0.25) (layer F.Cu) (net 6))
 (segment (start 74.92501 46.81182) (end 73.288191 45.175001) (width 0.25) (layer F.Cu) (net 6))
 (segment (start 76.6 59.5) (end 74.92501 57.82501) (width 0.25) (layer F.Cu) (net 6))
 (segment (start 78.1 59.5) (end 76.6 59.5) (width 0.25) (layer F.Cu) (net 6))
 (segment (start 78.6 70) (end 78.1 69.5) (width 0.25) (layer F.Cu) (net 8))
 (segment (start 81 70) (end 78.6 70) (width 0.25) (layer F.Cu) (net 8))
 (segment (start 64.475001 69.575001) (end 64.4 69.5) (width 0.25) (layer F.Cu) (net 14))
 (segment (start 64.4 69.5) (end 62.9 69.5) (width 0.25) (layer F.Cu) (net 14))
 (segment (start 74.914213 76) (end 80 76) (width 0.25) (layer F.Cu) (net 14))
 (segment (start 73.5 76) (end 74.914213 76) (width 0.25) (layer F.Cu) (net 14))
 (segment (start 65.985002 69.5) (end 62.9 69.5) (width 0.25) (layer F.Cu) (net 14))
 (segment (start 68.325001 71.839999) (end 65.985002 69.5) (width 0.25) (layer F.Cu) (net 14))
 (segment (start 68.325001 73.810003) (end 68.325001 71.839999) (width 0.25) (layer F.Cu) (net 14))
 (segment (start 70.514998 76) (end 68.325001 73.810003) (width 0.25) (layer F.Cu) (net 14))
 (segment (start 73.5 76) (end 70.514998 76) (width 0.25) (layer F.Cu) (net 14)))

